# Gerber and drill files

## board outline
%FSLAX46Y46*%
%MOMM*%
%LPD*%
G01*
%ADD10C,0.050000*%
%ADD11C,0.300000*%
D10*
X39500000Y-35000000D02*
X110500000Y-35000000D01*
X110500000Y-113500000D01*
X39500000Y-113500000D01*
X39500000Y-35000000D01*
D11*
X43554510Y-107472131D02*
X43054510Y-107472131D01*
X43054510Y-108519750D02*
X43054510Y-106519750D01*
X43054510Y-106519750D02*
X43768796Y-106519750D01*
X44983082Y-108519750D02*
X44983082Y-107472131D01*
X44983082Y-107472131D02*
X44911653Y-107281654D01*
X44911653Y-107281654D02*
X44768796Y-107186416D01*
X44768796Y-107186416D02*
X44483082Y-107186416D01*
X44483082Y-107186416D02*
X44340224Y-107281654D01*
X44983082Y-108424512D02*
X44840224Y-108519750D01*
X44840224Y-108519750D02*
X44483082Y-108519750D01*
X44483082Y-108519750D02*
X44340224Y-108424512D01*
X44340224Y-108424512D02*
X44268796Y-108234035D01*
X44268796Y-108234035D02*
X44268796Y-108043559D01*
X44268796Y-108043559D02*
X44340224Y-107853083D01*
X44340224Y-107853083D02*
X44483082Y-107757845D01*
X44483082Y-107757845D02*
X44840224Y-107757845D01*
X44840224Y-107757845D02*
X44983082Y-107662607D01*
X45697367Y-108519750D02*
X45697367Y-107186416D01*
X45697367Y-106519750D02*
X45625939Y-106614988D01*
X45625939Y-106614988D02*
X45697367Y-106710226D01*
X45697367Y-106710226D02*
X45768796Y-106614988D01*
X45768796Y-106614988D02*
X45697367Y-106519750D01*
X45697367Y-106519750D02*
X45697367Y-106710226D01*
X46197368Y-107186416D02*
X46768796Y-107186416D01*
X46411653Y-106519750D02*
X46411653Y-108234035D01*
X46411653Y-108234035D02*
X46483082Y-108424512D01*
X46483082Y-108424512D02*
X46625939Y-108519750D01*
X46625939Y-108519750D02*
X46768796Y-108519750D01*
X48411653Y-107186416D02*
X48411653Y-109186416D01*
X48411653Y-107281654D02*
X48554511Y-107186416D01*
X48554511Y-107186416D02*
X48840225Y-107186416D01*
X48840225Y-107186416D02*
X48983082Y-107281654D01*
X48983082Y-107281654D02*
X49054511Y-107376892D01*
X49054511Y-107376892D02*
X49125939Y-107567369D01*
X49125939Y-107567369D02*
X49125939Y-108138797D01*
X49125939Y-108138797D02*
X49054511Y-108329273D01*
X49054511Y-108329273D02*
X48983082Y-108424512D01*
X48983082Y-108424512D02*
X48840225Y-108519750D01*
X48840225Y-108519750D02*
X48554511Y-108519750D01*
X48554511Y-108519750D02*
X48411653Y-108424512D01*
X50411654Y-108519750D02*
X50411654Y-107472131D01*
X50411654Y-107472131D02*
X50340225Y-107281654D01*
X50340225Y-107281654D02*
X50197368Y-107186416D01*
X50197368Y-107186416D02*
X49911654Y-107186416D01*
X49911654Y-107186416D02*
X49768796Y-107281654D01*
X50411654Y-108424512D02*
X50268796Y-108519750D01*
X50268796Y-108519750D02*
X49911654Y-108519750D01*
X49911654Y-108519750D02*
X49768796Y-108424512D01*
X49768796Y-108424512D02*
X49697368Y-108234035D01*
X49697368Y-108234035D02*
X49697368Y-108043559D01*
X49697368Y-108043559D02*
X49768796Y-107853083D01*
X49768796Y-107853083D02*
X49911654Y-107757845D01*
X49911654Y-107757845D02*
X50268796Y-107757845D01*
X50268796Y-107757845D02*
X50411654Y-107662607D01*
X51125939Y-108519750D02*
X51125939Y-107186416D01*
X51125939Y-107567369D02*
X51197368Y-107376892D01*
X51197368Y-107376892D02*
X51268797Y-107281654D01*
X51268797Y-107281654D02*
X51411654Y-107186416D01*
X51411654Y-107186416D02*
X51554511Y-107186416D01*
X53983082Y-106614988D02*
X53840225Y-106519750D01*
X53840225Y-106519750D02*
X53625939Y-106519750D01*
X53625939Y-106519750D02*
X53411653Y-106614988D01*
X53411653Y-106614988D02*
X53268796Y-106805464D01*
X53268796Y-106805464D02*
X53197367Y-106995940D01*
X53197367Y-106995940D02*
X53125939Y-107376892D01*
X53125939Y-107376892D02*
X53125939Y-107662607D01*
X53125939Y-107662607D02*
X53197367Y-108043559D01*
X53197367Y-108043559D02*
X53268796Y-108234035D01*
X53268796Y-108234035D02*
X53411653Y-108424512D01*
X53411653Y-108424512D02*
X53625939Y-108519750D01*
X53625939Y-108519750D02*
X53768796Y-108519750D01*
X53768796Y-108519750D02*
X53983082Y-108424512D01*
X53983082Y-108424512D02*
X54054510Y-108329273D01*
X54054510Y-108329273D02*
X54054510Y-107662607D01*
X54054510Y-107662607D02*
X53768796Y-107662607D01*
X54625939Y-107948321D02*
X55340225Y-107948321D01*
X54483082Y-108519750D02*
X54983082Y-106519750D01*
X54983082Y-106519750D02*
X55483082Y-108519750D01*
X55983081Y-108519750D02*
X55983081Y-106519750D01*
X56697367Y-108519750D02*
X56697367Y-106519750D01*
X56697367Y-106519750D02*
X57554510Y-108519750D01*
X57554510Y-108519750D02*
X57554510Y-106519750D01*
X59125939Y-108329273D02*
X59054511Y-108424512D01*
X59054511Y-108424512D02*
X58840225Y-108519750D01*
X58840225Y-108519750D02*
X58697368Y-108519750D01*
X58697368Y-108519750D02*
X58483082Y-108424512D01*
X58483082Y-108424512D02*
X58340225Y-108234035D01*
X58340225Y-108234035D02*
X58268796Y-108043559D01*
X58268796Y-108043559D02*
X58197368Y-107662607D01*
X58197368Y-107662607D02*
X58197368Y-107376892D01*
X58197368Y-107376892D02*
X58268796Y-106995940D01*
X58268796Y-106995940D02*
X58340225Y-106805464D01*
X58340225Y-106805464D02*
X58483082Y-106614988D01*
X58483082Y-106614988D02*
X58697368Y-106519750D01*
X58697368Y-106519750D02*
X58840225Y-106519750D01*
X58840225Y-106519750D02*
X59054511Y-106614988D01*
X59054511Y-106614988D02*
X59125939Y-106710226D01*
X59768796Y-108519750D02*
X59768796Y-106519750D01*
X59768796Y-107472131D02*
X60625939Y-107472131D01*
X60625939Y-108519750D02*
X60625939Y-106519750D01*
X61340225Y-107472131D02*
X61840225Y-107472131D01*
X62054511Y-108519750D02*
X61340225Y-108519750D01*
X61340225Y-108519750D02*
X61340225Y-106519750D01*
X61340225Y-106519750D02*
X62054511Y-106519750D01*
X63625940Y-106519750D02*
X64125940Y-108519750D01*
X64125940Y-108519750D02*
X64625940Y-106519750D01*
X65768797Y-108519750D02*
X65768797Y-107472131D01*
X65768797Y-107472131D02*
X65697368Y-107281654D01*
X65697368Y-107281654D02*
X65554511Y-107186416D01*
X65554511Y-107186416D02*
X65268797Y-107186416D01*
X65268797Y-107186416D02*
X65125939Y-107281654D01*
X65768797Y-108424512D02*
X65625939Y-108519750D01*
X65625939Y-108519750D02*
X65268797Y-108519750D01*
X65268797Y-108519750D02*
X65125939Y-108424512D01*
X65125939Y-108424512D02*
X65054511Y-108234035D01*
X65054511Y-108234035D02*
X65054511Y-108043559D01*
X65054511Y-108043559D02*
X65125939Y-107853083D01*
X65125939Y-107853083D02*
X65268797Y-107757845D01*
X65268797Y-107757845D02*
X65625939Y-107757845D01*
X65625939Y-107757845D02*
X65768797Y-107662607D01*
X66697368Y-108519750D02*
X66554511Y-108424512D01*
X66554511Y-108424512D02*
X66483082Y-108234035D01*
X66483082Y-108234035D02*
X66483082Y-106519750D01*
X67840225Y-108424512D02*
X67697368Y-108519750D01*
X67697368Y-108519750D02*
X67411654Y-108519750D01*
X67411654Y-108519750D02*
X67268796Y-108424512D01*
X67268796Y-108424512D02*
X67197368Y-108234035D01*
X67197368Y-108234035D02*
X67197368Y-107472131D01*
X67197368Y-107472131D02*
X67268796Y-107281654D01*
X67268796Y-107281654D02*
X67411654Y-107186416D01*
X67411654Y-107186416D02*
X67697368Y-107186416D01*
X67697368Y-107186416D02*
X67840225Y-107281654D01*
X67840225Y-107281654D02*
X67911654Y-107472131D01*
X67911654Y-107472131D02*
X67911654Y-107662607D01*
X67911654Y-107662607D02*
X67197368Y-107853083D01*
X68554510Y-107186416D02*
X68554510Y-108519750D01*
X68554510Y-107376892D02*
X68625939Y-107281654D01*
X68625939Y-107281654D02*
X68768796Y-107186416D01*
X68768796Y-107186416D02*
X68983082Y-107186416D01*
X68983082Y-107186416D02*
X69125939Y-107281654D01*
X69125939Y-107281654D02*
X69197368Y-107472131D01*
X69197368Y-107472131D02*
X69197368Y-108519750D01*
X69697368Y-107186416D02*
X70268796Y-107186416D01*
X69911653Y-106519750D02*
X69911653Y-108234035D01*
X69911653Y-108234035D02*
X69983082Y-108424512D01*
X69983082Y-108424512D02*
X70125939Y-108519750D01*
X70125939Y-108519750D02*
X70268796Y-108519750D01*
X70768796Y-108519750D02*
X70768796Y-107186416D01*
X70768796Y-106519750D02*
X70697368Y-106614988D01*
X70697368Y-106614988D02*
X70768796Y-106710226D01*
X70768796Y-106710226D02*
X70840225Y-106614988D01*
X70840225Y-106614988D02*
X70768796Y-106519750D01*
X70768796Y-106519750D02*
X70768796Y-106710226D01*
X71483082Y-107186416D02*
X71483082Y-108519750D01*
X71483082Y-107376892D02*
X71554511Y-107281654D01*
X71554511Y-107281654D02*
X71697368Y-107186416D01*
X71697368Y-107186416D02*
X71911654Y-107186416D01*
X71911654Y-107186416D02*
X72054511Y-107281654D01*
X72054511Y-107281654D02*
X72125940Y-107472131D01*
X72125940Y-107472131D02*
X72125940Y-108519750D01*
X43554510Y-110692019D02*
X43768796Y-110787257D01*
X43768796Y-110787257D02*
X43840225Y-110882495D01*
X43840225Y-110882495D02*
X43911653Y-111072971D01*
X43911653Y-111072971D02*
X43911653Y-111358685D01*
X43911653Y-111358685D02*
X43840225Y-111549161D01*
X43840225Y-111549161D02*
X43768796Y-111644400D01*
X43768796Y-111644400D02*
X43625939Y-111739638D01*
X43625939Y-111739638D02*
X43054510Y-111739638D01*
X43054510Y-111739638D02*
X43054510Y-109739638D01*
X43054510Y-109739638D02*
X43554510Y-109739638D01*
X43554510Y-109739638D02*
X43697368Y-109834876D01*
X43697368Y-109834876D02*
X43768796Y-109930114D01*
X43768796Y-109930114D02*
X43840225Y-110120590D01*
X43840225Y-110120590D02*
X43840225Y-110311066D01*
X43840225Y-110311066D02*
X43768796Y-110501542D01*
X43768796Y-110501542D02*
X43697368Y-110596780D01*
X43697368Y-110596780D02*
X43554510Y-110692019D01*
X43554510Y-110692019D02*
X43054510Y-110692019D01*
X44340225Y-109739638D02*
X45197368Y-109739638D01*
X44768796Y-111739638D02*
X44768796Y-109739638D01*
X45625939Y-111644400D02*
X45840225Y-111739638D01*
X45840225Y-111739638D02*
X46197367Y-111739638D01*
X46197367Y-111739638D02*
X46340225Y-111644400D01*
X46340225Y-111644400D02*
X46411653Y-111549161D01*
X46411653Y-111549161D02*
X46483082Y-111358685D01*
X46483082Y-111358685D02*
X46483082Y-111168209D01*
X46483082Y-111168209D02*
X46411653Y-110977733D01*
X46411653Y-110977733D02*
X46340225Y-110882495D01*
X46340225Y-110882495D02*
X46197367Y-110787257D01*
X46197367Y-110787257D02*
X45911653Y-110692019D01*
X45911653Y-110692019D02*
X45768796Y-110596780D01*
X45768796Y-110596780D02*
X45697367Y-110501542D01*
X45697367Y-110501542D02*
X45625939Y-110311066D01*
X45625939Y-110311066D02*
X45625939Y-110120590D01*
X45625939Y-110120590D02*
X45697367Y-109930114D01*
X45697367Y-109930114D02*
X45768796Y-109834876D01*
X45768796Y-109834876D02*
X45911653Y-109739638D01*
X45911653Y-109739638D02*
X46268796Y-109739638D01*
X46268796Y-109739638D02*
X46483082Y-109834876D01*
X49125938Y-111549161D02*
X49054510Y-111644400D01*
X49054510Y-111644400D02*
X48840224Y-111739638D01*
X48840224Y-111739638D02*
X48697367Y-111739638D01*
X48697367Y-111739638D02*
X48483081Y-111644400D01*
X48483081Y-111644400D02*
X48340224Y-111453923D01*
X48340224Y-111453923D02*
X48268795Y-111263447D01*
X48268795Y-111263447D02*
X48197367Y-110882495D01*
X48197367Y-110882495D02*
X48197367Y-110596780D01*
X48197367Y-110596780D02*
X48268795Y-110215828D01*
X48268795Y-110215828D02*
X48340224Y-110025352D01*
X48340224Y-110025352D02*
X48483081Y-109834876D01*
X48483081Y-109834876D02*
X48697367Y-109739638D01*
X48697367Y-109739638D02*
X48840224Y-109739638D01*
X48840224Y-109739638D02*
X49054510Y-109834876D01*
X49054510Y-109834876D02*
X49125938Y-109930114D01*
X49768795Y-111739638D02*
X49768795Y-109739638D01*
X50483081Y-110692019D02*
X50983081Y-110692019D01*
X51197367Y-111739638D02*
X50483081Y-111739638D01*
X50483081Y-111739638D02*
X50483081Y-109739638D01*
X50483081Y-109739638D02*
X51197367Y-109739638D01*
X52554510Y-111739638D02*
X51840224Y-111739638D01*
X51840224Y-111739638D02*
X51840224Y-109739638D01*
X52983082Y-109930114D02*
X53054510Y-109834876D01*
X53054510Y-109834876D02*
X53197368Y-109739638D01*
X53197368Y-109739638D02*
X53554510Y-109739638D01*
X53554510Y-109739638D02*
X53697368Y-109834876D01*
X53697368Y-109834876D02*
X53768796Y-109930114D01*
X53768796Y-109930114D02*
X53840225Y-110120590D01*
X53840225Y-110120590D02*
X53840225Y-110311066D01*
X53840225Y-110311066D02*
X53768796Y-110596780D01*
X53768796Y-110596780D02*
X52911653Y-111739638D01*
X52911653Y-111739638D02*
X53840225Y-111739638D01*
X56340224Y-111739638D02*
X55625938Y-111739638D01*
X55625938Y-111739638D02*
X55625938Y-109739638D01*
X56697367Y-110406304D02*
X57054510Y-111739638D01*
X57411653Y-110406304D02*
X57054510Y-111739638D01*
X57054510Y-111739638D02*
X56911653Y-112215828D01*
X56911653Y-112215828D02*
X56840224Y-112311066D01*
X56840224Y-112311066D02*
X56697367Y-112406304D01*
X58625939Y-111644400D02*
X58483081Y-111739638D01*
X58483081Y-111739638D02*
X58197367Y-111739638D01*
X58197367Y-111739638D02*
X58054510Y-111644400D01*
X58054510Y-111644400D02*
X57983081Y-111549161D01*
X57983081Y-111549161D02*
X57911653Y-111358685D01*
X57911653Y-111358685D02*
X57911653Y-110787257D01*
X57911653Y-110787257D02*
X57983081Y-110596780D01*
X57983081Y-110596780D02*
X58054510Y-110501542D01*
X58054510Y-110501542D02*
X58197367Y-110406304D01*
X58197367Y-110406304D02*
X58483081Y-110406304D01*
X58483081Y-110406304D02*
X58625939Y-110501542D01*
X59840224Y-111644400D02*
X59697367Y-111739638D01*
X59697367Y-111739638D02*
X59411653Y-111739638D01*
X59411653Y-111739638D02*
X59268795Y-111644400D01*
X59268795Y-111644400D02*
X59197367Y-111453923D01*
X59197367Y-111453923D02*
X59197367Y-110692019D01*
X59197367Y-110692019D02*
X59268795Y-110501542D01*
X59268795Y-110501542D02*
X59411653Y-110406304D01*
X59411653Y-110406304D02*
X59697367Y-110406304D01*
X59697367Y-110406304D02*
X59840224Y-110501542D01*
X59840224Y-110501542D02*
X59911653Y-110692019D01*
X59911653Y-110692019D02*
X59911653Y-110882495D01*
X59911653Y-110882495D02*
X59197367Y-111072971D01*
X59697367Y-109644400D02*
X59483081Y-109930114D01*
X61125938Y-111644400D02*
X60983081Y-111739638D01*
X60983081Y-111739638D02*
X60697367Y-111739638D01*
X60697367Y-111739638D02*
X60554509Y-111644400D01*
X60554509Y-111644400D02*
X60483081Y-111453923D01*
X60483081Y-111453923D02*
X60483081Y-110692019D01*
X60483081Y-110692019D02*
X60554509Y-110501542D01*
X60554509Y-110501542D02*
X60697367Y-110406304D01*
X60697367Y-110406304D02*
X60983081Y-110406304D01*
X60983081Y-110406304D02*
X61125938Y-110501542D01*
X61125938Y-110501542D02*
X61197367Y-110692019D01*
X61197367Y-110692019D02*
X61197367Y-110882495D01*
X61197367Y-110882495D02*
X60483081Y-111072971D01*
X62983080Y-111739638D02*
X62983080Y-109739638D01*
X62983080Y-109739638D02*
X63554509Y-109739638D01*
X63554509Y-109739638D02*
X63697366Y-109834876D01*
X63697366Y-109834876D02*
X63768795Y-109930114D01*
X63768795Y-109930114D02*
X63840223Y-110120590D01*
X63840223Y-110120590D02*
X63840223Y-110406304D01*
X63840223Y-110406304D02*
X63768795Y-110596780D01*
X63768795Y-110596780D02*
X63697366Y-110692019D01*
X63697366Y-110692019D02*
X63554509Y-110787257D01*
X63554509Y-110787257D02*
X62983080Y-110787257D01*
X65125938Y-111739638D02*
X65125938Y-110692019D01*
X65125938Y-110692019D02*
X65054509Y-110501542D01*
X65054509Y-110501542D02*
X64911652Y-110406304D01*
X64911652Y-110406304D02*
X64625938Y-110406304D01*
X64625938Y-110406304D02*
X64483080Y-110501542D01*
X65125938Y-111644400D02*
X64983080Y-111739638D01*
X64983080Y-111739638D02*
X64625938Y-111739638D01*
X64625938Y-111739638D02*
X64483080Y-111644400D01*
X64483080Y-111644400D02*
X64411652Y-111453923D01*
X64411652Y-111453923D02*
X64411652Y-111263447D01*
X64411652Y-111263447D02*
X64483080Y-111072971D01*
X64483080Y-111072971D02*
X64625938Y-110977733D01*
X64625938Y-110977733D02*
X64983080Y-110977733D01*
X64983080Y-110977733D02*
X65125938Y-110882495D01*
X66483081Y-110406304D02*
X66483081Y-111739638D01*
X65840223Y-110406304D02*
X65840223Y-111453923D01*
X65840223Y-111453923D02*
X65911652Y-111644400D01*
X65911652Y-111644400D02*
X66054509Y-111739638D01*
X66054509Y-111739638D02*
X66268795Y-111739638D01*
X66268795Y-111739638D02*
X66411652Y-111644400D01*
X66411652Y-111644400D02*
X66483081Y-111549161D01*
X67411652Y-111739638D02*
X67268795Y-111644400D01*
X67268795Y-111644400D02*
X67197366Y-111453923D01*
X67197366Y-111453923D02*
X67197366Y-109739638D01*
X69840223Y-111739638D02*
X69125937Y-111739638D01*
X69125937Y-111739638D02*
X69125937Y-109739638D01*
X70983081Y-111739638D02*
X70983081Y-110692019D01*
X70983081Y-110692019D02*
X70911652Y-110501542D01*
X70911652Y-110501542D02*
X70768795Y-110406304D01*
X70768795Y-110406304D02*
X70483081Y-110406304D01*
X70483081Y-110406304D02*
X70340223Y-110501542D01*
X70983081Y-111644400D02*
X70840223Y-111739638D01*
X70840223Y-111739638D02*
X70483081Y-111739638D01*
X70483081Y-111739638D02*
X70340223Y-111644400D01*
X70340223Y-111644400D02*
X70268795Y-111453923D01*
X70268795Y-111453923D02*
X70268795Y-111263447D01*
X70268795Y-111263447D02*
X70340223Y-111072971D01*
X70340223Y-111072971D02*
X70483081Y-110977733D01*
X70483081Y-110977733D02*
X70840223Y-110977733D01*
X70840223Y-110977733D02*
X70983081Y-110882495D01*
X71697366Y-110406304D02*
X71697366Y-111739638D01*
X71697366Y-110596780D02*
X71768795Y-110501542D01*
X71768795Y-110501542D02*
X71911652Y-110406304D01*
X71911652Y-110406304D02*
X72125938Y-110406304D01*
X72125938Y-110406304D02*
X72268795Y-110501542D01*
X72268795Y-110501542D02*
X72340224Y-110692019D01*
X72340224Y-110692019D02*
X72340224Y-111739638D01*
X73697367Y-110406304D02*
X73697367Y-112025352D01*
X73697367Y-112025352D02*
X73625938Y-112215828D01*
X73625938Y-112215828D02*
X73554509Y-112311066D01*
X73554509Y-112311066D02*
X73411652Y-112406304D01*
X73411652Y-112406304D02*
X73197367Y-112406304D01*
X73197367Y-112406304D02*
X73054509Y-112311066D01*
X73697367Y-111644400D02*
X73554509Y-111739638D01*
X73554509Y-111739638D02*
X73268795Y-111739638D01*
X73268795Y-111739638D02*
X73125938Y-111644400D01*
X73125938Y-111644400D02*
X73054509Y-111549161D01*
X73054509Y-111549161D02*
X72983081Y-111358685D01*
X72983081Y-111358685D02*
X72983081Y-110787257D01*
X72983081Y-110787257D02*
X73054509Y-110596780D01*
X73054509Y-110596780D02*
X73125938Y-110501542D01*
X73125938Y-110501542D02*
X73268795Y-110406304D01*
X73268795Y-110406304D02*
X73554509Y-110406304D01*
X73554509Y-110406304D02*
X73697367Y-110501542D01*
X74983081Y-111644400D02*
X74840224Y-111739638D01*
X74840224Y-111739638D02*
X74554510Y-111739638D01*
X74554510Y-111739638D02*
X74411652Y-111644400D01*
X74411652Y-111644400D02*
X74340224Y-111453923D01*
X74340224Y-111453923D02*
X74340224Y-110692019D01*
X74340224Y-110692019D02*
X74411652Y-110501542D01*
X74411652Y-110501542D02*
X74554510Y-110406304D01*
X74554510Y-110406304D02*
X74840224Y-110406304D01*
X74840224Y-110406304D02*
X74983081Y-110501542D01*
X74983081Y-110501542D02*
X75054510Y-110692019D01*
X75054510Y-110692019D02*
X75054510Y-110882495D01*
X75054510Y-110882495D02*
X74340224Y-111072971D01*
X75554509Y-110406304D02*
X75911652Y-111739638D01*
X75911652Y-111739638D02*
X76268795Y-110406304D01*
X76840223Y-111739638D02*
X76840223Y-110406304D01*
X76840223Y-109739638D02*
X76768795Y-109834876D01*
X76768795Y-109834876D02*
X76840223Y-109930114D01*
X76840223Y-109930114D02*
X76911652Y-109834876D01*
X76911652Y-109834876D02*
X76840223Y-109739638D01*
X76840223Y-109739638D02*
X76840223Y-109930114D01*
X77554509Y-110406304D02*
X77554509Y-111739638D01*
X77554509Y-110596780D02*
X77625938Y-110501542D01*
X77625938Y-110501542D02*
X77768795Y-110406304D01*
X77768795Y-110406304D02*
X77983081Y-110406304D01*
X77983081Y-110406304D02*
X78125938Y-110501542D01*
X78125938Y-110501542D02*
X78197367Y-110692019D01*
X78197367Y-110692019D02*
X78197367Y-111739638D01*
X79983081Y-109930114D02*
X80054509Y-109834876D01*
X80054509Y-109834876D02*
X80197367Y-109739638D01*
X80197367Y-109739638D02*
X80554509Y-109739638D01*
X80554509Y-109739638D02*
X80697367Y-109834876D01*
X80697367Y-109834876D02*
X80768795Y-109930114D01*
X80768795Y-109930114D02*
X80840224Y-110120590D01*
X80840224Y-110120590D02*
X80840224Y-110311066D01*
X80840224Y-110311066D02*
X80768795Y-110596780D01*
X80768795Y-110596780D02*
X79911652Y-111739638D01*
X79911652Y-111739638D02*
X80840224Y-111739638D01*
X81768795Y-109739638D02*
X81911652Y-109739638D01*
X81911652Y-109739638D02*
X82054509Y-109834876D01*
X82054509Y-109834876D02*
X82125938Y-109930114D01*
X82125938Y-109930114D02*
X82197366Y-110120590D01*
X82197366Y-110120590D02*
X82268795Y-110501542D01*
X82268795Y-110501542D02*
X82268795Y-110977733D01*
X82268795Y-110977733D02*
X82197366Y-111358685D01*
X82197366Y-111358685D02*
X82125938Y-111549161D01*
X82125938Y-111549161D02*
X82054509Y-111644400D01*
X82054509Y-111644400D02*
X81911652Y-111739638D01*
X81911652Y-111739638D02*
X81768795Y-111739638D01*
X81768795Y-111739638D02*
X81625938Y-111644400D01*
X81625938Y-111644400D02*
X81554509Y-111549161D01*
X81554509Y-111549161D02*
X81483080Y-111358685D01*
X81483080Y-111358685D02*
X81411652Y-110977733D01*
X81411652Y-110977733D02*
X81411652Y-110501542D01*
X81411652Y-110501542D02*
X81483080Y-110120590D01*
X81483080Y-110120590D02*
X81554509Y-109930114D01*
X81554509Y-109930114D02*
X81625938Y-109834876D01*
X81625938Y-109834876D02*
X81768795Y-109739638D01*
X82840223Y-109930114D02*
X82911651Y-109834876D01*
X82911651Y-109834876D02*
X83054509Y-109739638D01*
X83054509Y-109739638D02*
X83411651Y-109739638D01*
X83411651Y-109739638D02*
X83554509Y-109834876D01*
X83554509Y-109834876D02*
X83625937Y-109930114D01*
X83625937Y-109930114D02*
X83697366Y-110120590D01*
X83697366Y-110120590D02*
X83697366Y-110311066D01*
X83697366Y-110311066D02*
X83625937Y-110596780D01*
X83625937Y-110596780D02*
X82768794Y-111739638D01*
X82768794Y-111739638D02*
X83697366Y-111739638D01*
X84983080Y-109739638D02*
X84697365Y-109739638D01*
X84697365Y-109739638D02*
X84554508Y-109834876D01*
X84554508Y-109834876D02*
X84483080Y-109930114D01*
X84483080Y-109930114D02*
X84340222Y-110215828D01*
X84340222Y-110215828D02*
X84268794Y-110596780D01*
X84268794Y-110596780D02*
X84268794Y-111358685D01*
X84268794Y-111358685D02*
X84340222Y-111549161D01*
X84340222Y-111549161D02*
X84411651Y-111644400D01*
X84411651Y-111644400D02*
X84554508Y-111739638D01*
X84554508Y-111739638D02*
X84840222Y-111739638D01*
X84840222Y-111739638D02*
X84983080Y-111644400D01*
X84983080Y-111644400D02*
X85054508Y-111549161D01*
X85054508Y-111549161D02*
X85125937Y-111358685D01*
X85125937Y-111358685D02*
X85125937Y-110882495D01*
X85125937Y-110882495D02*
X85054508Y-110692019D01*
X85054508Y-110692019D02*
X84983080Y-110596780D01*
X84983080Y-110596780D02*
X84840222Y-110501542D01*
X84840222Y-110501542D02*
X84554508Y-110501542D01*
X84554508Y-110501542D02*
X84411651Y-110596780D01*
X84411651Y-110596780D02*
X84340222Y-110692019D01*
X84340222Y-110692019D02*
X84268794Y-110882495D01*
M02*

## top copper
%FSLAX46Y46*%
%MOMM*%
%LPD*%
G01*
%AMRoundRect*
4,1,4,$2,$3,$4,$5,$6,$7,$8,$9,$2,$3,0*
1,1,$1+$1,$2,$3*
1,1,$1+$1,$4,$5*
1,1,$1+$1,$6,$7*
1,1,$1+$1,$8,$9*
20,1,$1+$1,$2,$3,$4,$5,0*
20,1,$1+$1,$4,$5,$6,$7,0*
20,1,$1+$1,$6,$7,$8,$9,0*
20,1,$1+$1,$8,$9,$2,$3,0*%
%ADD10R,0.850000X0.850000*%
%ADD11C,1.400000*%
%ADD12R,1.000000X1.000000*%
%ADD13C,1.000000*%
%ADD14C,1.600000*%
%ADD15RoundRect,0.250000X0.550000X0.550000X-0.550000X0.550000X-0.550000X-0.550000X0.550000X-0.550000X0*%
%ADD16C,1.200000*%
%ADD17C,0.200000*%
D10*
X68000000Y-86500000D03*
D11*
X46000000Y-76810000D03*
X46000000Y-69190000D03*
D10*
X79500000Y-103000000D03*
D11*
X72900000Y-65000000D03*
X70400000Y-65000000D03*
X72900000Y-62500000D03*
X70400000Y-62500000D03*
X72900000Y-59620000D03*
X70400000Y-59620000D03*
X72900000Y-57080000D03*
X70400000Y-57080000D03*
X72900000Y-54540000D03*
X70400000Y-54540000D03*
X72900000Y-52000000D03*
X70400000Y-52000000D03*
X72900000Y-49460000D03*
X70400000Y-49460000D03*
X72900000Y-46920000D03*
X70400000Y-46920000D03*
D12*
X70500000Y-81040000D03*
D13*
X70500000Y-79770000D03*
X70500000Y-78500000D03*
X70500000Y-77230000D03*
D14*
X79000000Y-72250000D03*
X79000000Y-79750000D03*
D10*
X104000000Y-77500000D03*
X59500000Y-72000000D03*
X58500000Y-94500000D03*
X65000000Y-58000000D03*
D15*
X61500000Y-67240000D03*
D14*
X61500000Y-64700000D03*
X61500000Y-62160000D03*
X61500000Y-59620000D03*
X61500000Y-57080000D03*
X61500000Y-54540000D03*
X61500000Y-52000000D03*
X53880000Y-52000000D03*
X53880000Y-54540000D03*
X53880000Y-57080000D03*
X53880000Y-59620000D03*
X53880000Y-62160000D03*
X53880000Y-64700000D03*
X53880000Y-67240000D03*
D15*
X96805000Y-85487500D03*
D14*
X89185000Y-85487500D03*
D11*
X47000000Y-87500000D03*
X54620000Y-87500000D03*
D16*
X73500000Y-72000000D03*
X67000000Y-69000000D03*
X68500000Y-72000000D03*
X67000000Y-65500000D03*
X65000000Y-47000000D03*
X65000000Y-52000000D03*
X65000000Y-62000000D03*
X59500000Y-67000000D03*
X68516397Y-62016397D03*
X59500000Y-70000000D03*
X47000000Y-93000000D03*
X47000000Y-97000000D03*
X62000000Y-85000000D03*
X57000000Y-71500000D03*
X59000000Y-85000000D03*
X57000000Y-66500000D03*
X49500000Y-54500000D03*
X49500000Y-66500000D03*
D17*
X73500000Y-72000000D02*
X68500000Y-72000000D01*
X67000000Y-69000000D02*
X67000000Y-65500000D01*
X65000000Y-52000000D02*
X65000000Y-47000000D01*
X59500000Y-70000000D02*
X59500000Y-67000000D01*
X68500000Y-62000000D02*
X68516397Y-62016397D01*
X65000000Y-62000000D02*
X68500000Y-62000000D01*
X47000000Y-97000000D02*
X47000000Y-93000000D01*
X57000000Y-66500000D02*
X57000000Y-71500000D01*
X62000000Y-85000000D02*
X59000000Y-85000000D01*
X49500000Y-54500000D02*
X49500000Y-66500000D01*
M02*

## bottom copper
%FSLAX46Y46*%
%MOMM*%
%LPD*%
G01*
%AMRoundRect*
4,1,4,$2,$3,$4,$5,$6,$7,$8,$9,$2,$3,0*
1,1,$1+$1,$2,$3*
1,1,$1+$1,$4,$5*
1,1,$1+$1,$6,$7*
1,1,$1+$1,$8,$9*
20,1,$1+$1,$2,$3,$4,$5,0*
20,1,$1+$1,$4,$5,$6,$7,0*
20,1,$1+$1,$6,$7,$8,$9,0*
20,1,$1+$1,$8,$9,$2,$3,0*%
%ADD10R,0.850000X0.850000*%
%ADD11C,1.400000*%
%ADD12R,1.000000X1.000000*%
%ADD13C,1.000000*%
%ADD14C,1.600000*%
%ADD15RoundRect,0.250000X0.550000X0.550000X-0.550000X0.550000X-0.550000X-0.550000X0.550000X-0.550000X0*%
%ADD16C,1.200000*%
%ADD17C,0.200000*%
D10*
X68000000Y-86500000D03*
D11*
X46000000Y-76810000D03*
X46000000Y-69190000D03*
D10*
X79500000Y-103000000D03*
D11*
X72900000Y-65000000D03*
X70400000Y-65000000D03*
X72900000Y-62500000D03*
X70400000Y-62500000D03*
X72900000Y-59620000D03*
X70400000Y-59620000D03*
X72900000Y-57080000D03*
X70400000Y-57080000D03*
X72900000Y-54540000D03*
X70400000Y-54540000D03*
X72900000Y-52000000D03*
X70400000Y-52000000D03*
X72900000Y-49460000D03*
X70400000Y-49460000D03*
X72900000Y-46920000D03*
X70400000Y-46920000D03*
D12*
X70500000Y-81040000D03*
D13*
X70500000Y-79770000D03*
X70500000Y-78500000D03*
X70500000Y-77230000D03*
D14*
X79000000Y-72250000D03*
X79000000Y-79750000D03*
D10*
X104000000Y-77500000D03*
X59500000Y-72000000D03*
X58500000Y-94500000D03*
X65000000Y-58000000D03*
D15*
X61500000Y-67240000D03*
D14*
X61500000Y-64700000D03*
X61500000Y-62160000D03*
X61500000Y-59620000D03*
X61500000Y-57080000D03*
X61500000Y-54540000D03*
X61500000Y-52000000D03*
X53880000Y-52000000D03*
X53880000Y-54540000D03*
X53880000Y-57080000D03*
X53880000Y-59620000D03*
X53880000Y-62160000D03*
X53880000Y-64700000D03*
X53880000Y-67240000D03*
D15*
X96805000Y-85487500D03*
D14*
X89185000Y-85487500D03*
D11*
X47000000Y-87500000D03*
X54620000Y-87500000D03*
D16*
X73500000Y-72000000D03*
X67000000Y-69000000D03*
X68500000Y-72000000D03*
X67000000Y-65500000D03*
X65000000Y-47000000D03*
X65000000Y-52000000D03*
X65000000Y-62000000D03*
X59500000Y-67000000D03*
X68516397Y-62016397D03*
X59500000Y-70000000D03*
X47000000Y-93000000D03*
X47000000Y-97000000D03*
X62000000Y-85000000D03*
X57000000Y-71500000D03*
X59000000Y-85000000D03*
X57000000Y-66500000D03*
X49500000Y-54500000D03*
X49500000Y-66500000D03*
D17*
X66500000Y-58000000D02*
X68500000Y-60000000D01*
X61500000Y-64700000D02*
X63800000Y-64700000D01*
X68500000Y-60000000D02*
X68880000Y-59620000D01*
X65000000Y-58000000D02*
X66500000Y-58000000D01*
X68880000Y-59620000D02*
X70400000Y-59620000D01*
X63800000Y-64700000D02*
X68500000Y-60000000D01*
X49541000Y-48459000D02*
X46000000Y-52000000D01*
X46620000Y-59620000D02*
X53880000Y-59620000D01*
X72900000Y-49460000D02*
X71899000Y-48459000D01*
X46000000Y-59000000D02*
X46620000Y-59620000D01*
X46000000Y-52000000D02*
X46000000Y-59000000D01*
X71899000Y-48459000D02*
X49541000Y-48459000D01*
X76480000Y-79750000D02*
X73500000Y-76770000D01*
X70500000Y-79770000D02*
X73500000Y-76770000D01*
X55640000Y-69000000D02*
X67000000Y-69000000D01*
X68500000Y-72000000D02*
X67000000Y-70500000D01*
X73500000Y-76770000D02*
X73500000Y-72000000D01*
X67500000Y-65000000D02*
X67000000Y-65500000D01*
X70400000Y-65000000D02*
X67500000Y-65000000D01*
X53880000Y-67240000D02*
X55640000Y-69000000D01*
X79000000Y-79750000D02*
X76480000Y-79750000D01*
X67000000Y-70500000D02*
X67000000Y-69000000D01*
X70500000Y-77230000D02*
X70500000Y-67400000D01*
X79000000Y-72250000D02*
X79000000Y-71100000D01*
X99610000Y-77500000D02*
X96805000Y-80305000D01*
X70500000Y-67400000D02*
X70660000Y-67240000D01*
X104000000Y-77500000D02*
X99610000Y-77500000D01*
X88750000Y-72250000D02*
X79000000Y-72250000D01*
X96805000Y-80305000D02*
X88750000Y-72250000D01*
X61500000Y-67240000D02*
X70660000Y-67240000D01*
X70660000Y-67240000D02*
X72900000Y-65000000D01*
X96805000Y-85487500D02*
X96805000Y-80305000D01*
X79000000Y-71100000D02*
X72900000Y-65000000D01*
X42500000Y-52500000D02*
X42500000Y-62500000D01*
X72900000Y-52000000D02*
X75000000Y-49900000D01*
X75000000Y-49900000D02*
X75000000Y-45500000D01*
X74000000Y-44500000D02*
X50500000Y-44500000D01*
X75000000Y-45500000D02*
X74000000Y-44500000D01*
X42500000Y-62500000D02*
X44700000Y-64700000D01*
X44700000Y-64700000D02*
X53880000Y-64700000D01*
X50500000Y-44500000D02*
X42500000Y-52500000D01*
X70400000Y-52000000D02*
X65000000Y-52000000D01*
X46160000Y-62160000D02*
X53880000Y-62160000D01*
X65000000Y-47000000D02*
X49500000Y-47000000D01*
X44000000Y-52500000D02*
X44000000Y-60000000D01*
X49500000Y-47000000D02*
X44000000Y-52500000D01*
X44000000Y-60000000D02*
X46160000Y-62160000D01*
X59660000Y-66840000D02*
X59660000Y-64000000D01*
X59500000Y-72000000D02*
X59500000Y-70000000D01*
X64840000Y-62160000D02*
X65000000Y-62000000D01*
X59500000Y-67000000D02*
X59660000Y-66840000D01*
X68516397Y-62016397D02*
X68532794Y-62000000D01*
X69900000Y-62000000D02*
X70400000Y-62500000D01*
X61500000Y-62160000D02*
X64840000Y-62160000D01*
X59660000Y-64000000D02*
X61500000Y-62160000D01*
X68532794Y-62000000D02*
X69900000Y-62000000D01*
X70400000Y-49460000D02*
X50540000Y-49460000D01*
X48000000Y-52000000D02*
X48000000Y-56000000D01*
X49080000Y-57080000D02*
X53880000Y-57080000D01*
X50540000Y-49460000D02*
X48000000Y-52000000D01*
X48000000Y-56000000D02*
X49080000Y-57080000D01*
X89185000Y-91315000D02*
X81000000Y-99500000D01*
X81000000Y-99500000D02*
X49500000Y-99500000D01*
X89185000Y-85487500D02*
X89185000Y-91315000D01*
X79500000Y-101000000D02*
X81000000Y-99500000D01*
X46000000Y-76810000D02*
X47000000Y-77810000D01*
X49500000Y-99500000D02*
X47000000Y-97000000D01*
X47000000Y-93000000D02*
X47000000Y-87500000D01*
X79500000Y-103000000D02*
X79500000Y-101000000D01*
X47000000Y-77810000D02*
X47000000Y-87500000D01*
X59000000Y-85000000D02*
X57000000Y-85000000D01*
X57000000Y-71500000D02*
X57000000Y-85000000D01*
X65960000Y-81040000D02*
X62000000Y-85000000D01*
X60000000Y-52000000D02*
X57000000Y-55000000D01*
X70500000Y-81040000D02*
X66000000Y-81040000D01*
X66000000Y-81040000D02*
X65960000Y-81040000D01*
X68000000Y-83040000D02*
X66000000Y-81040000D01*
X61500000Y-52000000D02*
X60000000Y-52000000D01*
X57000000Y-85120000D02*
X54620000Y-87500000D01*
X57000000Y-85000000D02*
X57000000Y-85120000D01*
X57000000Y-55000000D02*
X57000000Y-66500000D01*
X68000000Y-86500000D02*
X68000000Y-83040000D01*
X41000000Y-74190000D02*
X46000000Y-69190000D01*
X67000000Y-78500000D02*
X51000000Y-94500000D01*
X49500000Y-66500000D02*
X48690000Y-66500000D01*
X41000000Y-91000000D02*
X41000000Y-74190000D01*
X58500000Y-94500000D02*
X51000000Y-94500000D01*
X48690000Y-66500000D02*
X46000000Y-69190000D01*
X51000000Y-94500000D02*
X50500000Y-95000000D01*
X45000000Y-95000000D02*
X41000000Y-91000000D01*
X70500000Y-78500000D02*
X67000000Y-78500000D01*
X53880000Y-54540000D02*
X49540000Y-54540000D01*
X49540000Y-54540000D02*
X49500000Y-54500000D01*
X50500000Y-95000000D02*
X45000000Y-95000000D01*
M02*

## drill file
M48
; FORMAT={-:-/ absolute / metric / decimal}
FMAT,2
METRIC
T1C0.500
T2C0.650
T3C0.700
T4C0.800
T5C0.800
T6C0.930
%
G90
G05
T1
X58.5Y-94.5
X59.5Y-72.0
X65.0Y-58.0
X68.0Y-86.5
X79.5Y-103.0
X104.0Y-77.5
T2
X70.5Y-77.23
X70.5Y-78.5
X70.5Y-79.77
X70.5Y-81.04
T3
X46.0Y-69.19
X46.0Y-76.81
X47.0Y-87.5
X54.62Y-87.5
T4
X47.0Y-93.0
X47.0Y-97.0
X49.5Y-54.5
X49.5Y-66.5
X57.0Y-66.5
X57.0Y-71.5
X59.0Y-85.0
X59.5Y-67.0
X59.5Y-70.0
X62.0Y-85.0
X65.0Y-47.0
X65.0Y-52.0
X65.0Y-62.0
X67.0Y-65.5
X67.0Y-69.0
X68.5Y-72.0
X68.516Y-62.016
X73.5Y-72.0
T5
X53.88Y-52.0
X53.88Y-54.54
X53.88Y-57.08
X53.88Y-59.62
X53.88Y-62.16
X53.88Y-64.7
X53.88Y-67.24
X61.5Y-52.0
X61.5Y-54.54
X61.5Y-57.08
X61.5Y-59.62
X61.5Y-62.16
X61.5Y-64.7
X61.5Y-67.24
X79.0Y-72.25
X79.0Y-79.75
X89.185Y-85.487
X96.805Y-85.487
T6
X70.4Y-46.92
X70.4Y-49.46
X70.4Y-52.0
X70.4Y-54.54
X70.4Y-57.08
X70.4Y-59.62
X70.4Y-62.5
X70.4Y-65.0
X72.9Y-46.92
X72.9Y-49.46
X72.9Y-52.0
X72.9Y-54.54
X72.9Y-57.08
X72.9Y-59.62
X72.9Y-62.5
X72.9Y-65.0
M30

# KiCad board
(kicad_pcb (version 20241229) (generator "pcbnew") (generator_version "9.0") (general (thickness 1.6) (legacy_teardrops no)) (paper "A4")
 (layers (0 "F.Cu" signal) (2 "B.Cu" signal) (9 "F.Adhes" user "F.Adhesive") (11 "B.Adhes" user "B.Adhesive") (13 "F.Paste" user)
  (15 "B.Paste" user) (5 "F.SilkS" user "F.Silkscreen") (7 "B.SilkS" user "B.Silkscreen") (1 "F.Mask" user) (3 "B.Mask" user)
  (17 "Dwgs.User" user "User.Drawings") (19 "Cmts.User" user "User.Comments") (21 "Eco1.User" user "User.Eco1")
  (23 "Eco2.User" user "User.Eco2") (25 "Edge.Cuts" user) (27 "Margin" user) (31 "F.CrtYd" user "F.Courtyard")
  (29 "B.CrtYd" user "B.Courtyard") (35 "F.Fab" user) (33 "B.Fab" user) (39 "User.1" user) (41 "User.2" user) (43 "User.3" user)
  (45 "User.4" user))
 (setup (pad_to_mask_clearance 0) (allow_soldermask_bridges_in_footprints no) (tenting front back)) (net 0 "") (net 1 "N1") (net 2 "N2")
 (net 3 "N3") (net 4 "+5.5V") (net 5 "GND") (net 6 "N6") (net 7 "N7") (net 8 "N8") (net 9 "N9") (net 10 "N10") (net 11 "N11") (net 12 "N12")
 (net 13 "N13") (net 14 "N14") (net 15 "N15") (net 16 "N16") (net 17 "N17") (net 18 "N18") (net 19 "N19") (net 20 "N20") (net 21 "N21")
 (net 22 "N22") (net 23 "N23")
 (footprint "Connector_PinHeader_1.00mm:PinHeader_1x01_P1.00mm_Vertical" (layer "F.Cu") (at 68 86.5 180)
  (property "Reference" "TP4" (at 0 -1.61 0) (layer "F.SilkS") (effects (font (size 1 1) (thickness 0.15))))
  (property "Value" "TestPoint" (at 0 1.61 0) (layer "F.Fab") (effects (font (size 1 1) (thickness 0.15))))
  (pad "1" thru_hole rect (at 0 0 180) (size 0.85 0.85) (drill 0.5) (layers "*.Cu" "*.Mask") (remove_unused_layers no) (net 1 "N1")))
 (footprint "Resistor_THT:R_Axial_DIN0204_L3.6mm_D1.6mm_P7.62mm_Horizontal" (layer "F.Cu") (at 46 76.81 90)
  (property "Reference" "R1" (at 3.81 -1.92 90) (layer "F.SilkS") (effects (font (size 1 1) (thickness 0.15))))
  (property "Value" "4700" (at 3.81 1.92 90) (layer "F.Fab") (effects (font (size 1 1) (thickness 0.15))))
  (pad "1" thru_hole circle (at 0 0 90) (size 1.4 1.4) (drill 0.7) (layers "*.Cu" "*.Mask") (remove_unused_layers no) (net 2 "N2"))
  (pad "2" thru_hole circle (at 7.62 0 90) (size 1.4 1.4) (drill 0.7) (layers "*.Cu" "*.Mask") (remove_unused_layers no) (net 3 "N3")))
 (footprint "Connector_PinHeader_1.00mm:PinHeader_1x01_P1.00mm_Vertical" (layer "F.Cu") (at 79.5 103 180)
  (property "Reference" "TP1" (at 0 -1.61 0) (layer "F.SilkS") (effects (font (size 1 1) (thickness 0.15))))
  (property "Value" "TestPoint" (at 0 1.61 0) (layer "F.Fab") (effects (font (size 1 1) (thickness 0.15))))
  (pad "1" thru_hole rect (at 0 0 180) (size 0.85 0.85) (drill 0.5) (layers "*.Cu" "*.Mask") (remove_unused_layers no) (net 2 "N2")))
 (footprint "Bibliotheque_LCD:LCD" (layer "F.Cu") (at 111 53.5)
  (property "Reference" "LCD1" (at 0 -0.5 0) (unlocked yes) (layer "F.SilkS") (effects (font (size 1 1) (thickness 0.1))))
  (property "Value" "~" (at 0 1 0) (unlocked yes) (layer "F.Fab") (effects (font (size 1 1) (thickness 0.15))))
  (pad "1" thru_hole circle (at -38.1 11.5 270) (size 1.4 1.4) (drill 0.93) (layers "*.Cu" "*.Mask") (remove_unused_layers no)
   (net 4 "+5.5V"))
  (pad "2" thru_hole circle (at -40.6 11.5 270) (size 1.4 1.4) (drill 0.93) (layers "*.Cu" "*.Mask") (remove_unused_layers no) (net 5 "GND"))
  (pad "3" thru_hole circle (at -38.1 9 270) (size 1.4 1.4) (drill 0.93) (layers "*.Cu" "*.Mask") (remove_unused_layers no) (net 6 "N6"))
  (pad "4" thru_hole circle (at -40.6 9 270) (size 1.4 1.4) (drill 0.93) (layers "*.Cu" "*.Mask") (remove_unused_layers no) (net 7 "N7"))
  (pad "5" thru_hole circle (at -38.1 6.12 270) (size 1.4 1.4) (drill 0.93) (layers "*.Cu" "*.Mask") (remove_unused_layers no) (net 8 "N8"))
  (pad "6" thru_hole circle (at -40.6 6.12 270) (size 1.4 1.4) (drill 0.93) (layers "*.Cu" "*.Mask") (remove_unused_layers no) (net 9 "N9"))
  (pad "7" thru_hole circle (at -38.1 3.58 270) (size 1.4 1.4) (drill 0.93) (layers "*.Cu" "*.Mask") (remove_unused_layers no)
   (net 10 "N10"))
  (pad "8" thru_hole circle (at -40.6 3.58 270) (size 1.4 1.4) (drill 0.93) (layers "*.Cu" "*.Mask") (remove_unused_layers no)
   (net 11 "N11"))
  (pad "9" thru_hole circle (at -38.1 1.04 270) (size 1.4 1.4) (drill 0.93) (layers "*.Cu" "*.Mask") (remove_unused_layers no)
   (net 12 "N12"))
  (pad "10" thru_hole circle (at -40.6 1.04 270) (size 1.4 1.4) (drill 0.93) (layers "*.Cu" "*.Mask") (remove_unused_layers no)
   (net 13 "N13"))
  (pad "11" thru_hole circle (at -38.1 -1.5 270) (size 1.4 1.4) (drill 0.93) (layers "*.Cu" "*.Mask") (remove_unused_layers no)
   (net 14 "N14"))
  (pad "12" thru_hole circle (at -40.6 -1.5 270) (size 1.4 1.4) (drill 0.93) (layers "*.Cu" "*.Mask") (remove_unused_layers no)
   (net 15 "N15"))
  (pad "13" thru_hole circle (at -38.1 -4.04 270) (size 1.4 1.4) (drill 0.93) (layers "*.Cu" "*.Mask") (remove_unused_layers no)
   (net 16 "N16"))
  (pad "14" thru_hole circle (at -40.6 -4.04 270) (size 1.4 1.4) (drill 0.93) (layers "*.Cu" "*.Mask") (remove_unused_layers no)
   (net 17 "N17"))
  (pad "15" thru_hole circle (at -38.1 -6.58 270) (size 1.4 1.4) (drill 0.93) (layers "*.Cu" "*.Mask") (remove_unused_layers no)
   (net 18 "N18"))
  (pad "16" thru_hole circle (at -40.6 -6.58 270) (size 1.4 1.4) (drill 0.93) (layers "*.Cu" "*.Mask") (remove_unused_layers no)
   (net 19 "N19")))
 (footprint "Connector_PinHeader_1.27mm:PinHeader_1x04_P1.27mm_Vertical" (layer "F.Cu") (at 70.5 81.04 180)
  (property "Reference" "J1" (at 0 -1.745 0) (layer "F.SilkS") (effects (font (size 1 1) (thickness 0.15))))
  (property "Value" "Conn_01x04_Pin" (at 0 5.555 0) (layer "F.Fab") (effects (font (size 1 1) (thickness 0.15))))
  (pad "1" thru_hole rect (at 0 0 180) (size 1 1) (drill 0.65) (layers "*.Cu" "*.Mask") (remove_unused_layers no) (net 1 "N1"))
  (pad "2" thru_hole circle (at 0 1.27 180) (size 1 1) (drill 0.65) (layers "*.Cu" "*.Mask") (remove_unused_layers no) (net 5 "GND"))
  (pad "3" thru_hole circle (at 0 2.54 180) (size 1 1) (drill 0.65) (layers "*.Cu" "*.Mask") (remove_unused_layers no) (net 3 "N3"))
  (pad "4" thru_hole circle (at 0 3.81 180) (size 1 1) (drill 0.65) (layers "*.Cu" "*.Mask") (remove_unused_layers no) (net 4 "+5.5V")))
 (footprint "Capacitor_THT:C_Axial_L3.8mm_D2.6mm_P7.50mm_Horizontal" (layer "F.Cu") (at 79 72.25 -90)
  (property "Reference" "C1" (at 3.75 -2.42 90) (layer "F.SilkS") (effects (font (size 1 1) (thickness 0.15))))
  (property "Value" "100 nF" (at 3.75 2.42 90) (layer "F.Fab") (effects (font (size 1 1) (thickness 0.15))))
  (pad "1" thru_hole circle (at 0 0 270) (size 1.6 1.6) (drill 0.8) (layers "*.Cu" "*.Mask") (remove_unused_layers no) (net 4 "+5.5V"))
  (pad "2" thru_hole circle (at 7.5 0 270) (size 1.6 1.6) (drill 0.8) (layers "*.Cu" "*.Mask") (remove_unused_layers no) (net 5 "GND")))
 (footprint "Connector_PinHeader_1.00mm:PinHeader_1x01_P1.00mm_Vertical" (layer "F.Cu") (at 104 77.5 180)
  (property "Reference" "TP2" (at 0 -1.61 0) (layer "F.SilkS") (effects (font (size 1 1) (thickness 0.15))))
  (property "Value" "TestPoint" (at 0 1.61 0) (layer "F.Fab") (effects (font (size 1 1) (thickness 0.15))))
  (pad "1" thru_hole rect (at 0 0 180) (size 0.85 0.85) (drill 0.5) (layers "*.Cu" "*.Mask") (remove_unused_layers no) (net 4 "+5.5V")))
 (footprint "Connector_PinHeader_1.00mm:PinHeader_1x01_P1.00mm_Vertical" (layer "F.Cu") (at 59.5 72 180)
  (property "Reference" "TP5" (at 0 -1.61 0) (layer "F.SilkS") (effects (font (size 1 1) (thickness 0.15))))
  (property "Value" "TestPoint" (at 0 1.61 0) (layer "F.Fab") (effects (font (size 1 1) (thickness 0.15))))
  (pad "1" thru_hole rect (at 0 0 180) (size 0.85 0.85) (drill 0.5) (layers "*.Cu" "*.Mask") (remove_unused_layers no) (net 7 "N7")))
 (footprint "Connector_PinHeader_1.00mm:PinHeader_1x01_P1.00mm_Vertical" (layer "F.Cu") (at 58.5 94.5)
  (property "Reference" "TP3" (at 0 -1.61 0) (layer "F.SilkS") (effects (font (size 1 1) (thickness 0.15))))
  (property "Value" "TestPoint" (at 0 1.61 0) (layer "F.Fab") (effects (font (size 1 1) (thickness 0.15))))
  (pad "1" thru_hole rect (at 0 0) (size 0.85 0.85) (drill 0.5) (layers "*.Cu" "*.Mask") (remove_unused_layers no) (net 3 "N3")))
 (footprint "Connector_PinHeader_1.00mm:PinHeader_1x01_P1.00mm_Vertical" (layer "F.Cu") (at 65 58 180)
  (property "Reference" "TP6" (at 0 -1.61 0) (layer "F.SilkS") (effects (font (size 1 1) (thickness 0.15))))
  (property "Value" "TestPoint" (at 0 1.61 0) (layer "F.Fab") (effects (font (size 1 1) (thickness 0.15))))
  (pad "1" thru_hole rect (at 0 0 180) (size 0.85 0.85) (drill 0.5) (layers "*.Cu" "*.Mask") (remove_unused_layers no) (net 9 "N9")))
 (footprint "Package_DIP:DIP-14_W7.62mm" (layer "F.Cu") (at 61.5 67.24 180)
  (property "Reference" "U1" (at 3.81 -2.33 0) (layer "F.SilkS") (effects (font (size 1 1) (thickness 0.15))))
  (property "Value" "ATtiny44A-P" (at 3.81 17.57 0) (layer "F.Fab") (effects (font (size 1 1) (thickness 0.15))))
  (pad "1" thru_hole roundrect (at 0 0 180) (size 1.6 1.6) (drill 0.8) (layers "*.Cu" "*.Mask") (remove_unused_layers no)
   (roundrect_rratio 0.15625) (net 4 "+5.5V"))
  (pad "2" thru_hole circle (at 0 2.54 180) (size 1.6 1.6) (drill 0.8) (layers "*.Cu" "*.Mask") (remove_unused_layers no) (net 9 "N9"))
  (pad "3" thru_hole circle (at 0 5.08 180) (size 1.6 1.6) (drill 0.8) (layers "*.Cu" "*.Mask") (remove_unused_layers no) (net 7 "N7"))
  (pad "4" thru_hole circle (at 0 7.62 180) (size 1.6 1.6) (drill 0.8) (layers "*.Cu" "*.Mask") (remove_unused_layers no) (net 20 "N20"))
  (pad "5" thru_hole circle (at 0 10.16 180) (size 1.6 1.6) (drill 0.8) (layers "*.Cu" "*.Mask") (remove_unused_layers no) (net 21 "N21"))
  (pad "6" thru_hole circle (at 0 12.7 180) (size 1.6 1.6) (drill 0.8) (layers "*.Cu" "*.Mask") (remove_unused_layers no) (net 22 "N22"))
  (pad "7" thru_hole circle (at 0 15.24 180) (size 1.6 1.6) (drill 0.8) (layers "*.Cu" "*.Mask") (remove_unused_layers no) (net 1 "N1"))
  (pad "8" thru_hole circle (at 7.62 15.24 180) (size 1.6 1.6) (drill 0.8) (layers "*.Cu" "*.Mask") (remove_unused_layers no) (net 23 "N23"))
  (pad "9" thru_hole circle (at 7.62 12.7 180) (size 1.6 1.6) (drill 0.8) (layers "*.Cu" "*.Mask") (remove_unused_layers no) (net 3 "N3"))
  (pad "10" thru_hole circle (at 7.62 10.16 180) (size 1.6 1.6) (drill 0.8) (layers "*.Cu" "*.Mask") (remove_unused_layers no)
   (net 17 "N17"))
  (pad "11" thru_hole circle (at 7.62 7.62 180) (size 1.6 1.6) (drill 0.8) (layers "*.Cu" "*.Mask") (remove_unused_layers no) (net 16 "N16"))
  (pad "12" thru_hole circle (at 7.62 5.08 180) (size 1.6 1.6) (drill 0.8) (layers "*.Cu" "*.Mask") (remove_unused_layers no) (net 15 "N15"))
  (pad "13" thru_hole circle (at 7.62 2.54 180) (size 1.6 1.6) (drill 0.8) (layers "*.Cu" "*.Mask") (remove_unused_layers no) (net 14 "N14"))
  (pad "14" thru_hole circle (at 7.62 0 180) (size 1.6 1.6) (drill 0.8) (layers "*.Cu" "*.Mask") (remove_unused_layers no) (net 5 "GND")))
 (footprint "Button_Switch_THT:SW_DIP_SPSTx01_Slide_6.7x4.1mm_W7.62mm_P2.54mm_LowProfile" (layer "F.Cu") (at 96.805 85.4875 180)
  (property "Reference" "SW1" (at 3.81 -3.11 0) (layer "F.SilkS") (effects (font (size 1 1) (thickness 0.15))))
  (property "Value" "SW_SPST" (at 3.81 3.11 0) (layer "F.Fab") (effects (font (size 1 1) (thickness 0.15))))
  (pad "1" thru_hole roundrect (at 0 0 180) (size 1.6 1.6) (drill 0.8) (layers "*.Cu" "*.Mask") (remove_unused_layers no)
   (roundrect_rratio 0.15625) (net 4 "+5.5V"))
  (pad "2" thru_hole circle (at 7.62 0 180) (size 1.6 1.6) (drill 0.8) (layers "*.Cu" "*.Mask") (remove_unused_layers no) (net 2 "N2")))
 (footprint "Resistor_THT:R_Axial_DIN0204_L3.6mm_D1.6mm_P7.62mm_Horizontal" (layer "F.Cu") (at 47 87.5)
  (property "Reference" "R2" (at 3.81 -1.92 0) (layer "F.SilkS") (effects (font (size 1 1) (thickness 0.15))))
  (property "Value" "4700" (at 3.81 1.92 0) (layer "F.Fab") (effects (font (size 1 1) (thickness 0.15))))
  (pad "1" thru_hole circle (at 0 0) (size 1.4 1.4) (drill 0.7) (layers "*.Cu" "*.Mask") (remove_unused_layers no) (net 2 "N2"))
  (pad "2" thru_hole circle (at 7.62 0) (size 1.4 1.4) (drill 0.7) (layers "*.Cu" "*.Mask") (remove_unused_layers no) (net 1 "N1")))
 (gr_rect (start 39.5 35) (end 110.5 113.5) (stroke (width 0.05) (type default)) (fill no) (layer "Edge.Cuts"))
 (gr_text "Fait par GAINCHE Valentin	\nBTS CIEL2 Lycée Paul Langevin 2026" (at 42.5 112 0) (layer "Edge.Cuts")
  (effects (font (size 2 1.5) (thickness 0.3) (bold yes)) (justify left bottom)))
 (segment (start 66.5 58) (end 68.5 60) (width 0.2) (layer "B.Cu") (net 9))
 (segment (start 61.5 64.7) (end 63.8 64.7) (width 0.2) (layer "B.Cu") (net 9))
 (segment (start 68.5 60) (end 68.88 59.62) (width 0.2) (layer "B.Cu") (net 9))
 (segment (start 65 58) (end 66.5 58) (width 0.2) (layer "B.Cu") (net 9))
 (segment (start 68.88 59.62) (end 70.4 59.62) (width 0.2) (layer "B.Cu") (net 9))
 (segment (start 63.8 64.7) (end 68.5 60) (width 0.2) (layer "B.Cu") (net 9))
 (segment (start 49.541 48.459) (end 46 52) (width 0.2) (layer "B.Cu") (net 16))
 (segment (start 46.62 59.62) (end 53.88 59.62) (width 0.2) (layer "B.Cu") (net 16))
 (segment (start 72.9 49.46) (end 71.899 48.459) (width 0.2) (layer "B.Cu") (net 16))
 (segment (start 46 59) (end 46.62 59.62) (width 0.2) (layer "B.Cu") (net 16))
 (segment (start 46 52) (end 46 59) (width 0.2) (layer "B.Cu") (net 16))
 (segment (start 71.899 48.459) (end 49.541 48.459) (width 0.2) (layer "B.Cu") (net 16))
 (segment (start 73.5 72) (end 68.5 72) (width 0.2) (layer "F.Cu") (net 5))
 (segment (start 67 69) (end 67 65.5) (width 0.2) (layer "F.Cu") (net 5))
 (via (at 73.5 72) (size 1.2) (drill 0.8) (layers "F.Cu" "B.Cu") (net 5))
 (via (at 67 69) (size 1.2) (drill 0.8) (layers "F.Cu" "B.Cu") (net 5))
 (via (at 68.5 72) (size 1.2) (drill 0.8) (layers "F.Cu" "B.Cu") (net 5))
 (via (at 67 65.5) (size 1.2) (drill 0.8) (layers "F.Cu" "B.Cu") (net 5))
 (segment (start 76.48 79.75) (end 73.5 76.77) (width 0.2) (layer "B.Cu") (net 5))
 (segment (start 70.5 79.77) (end 73.5 76.77) (width 0.2) (layer "B.Cu") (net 5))
 (segment (start 55.64 69) (end 67 69) (width 0.2) (layer "B.Cu") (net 5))
 (segment (start 68.5 72) (end 67 70.5) (width 0.2) (layer "B.Cu") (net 5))
 (segment (start 73.5 76.77) (end 73.5 72) (width 0.2) (layer "B.Cu") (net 5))
 (segment (start 67.5 65) (end 67 65.5) (width 0.2) (layer "B.Cu") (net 5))
 (segment (start 70.4 65) (end 67.5 65) (width 0.2) (layer "B.Cu") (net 5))
 (segment (start 53.88 67.24) (end 55.64 69) (width 0.2) (layer "B.Cu") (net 5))
 (segment (start 79 79.75) (end 76.48 79.75) (width 0.2) (layer "B.Cu") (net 5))
 (segment (start 67 70.5) (end 67 69) (width 0.2) (layer "B.Cu") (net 5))
 (segment (start 70.5 77.23) (end 70.5 67.4) (width 0.2) (layer "B.Cu") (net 4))
 (segment (start 79 72.25) (end 79 71.1) (width 0.2) (layer "B.Cu") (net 4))
 (segment (start 99.61 77.5) (end 96.805 80.305) (width 0.2) (layer "B.Cu") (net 4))
 (segment (start 70.5 67.4) (end 70.66 67.24) (width 0.2) (layer "B.Cu") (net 4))
 (segment (start 104 77.5) (end 99.61 77.5) (width 0.2) (layer "B.Cu") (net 4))
 (segment (start 88.75 72.25) (end 79 72.25) (width 0.2) (layer "B.Cu") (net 4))
 (segment (start 96.805 80.305) (end 88.75 72.25) (width 0.2) (layer "B.Cu") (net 4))
 (segment (start 61.5 67.24) (end 70.66 67.24) (width 0.2) (layer "B.Cu") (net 4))
 (segment (start 70.66 67.24) (end 72.9 65) (width 0.2) (layer "B.Cu") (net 4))
 (segment (start 96.805 85.4875) (end 96.805 80.305) (width 0.2) (layer "B.Cu") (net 4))
 (segment (start 79 71.1) (end 72.9 65) (width 0.2) (layer "B.Cu") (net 4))
 (segment (start 42.5 52.5) (end 42.5 62.5) (width 0.2) (layer "B.Cu") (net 14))
 (segment (start 72.9 52) (end 75 49.9) (width 0.2) (layer "B.Cu") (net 14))
 (segment (start 75 49.9) (end 75 45.5) (width 0.2) (layer "B.Cu") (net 14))
 (segment (start 74 44.5) (end 50.5 44.5) (width 0.2) (layer "B.Cu") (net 14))
 (segment (start 75 45.5) (end 74 44.5) (width 0.2) (layer "B.Cu") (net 14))
 (segment (start 42.5 62.5) (end 44.7 64.7) (width 0.2) (layer "B.Cu") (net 14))
 (segment (start 44.7 64.7) (end 53.88 64.7) (width 0.2) (layer "B.Cu") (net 14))
 (segment (start 50.5 44.5) (end 42.5 52.5) (width 0.2) (layer "B.Cu") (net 14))
 (segment (start 65 52) (end 65 47) (width 0.2) (layer "F.Cu") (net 15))
 (via (at 65 47) (size 1.2) (drill 0.8) (layers "F.Cu" "B.Cu") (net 15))
 (via (at 65 52) (size 1.2) (drill 0.8) (layers "F.Cu" "B.Cu") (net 15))
 (segment (start 70.4 52) (end 65 52) (width 0.2) (layer "B.Cu") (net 15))
 (segment (start 46.16 62.16) (end 53.88 62.16) (width 0.2) (layer "B.Cu") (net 15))
 (segment (start 65 47) (end 49.5 47) (width 0.2) (layer "B.Cu") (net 15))
 (segment (start 44 52.5) (end 44 60) (width 0.2) (layer "B.Cu") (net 15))
 (segment (start 49.5 47) (end 44 52.5) (width 0.2) (layer "B.Cu") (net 15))
 (segment (start 44 60) (end 46.16 62.16) (width 0.2) (layer "B.Cu") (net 15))
 (segment (start 59.5 70) (end 59.5 67) (width 0.2) (layer "F.Cu") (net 7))
 (segment (start 68.5 62) (end 68.516397 62.016397) (width 0.2) (layer "F.Cu") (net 7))
 (segment (start 65 62) (end 68.5 62) (width 0.2) (layer "F.Cu") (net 7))
 (via (at 65 62) (size 1.2) (drill 0.8) (layers "F.Cu" "B.Cu") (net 7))
 (via (at 59.5 67) (size 1.2) (drill 0.8) (layers "F.Cu" "B.Cu") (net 7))
 (via (at 68.516397 62.016397) (size 1.2) (drill 0.8) (layers "F.Cu" "B.Cu") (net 7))
 (via (at 59.5 70) (size 1.2) (drill 0.8) (layers "F.Cu" "B.Cu") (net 7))
 (segment (start 59.66 66.84) (end 59.66 64) (width 0.2) (layer "B.Cu") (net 7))
 (segment (start 59.5 72) (end 59.5 70) (width 0.2) (layer "B.Cu") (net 7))
 (segment (start 64.84 62.16) (end 65 62) (width 0.2) (layer "B.Cu") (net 7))
 (segment (start 59.5 67) (end 59.66 66.84) (width 0.2) (layer "B.Cu") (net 7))
 (segment (start 68.516397 62.016397) (end 68.532794 62) (width 0.2) (layer "B.Cu") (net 7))
 (segment (start 69.9 62) (end 70.4 62.5) (width 0.2) (layer "B.Cu") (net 7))
 (segment (start 61.5 62.16) (end 64.84 62.16) (width 0.2) (layer "B.Cu") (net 7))
 (segment (start 59.66 64) (end 61.5 62.16) (width 0.2) (layer "B.Cu") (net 7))
 (segment (start 68.532794 62) (end 69.9 62) (width 0.2) (layer "B.Cu") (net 7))
 (segment (start 70.4 49.46) (end 50.54 49.46) (width 0.2) (layer "B.Cu") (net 17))
 (segment (start 48 52) (end 48 56) (width 0.2) (layer "B.Cu") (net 17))
 (segment (start 49.08 57.08) (end 53.88 57.08) (width 0.2) (layer "B.Cu") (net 17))
 (segment (start 50.54 49.46) (end 48 52) (width 0.2) (layer "B.Cu") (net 17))
 (segment (start 48 56) (end 49.08 57.08) (width 0.2) (layer "B.Cu") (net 17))
 (segment (start 47 97) (end 47 93) (width 0.2) (layer "F.Cu") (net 2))
 (via (at 47 93) (size 1.2) (drill 0.8) (layers "F.Cu" "B.Cu") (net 2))
 (via (at 47 97) (size 1.2) (drill 0.8) (layers "F.Cu" "B.Cu") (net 2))
 (segment (start 89.185 91.315) (end 81 99.5) (width 0.2) (layer "B.Cu") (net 2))
 (segment (start 81 99.5) (end 49.5 99.5) (width 0.2) (layer "B.Cu") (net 2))
 (segment (start 89.185 85.4875) (end 89.185 91.315) (width 0.2) (layer "B.Cu") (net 2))
 (segment (start 79.5 101) (end 81 99.5) (width 0.2) (layer "B.Cu") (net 2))
 (segment (start 46 76.81) (end 47 77.81) (width 0.2) (layer "B.Cu") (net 2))
 (segment (start 49.5 99.5) (end 47 97) (width 0.2) (layer "B.Cu") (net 2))
 (segment (start 47 93) (end 47 87.5) (width 0.2) (layer "B.Cu") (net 2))
 (segment (start 79.5 103) (end 79.5 101) (width 0.2) (layer "B.Cu") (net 2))
 (segment (start 47 77.81) (end 47 87.5) (width 0.2) (layer "B.Cu") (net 2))
 (segment (start 57 66.5) (end 57 71.5) (width 0.2) (layer "F.Cu") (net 1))
 (segment (start 62 85) (end 59 85) (width 0.2) (layer "F.Cu") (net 1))
 (via (at 62 85) (size 1.2) (drill 0.8) (layers "F.Cu" "B.Cu") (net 1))
 (via (at 57 71.5) (size 1.2) (drill 0.8) (layers "F.Cu" "B.Cu") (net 1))
 (via (at 59 85) (size 1.2) (drill 0.8) (layers "F.Cu" "B.Cu") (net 1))
 (via (at 57 66.5) (size 1.2) (drill 0.8) (layers "F.Cu" "B.Cu") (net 1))
 (segment (start 59 85) (end 57 85) (width 0.2) (layer "B.Cu") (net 1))
 (segment (start 57 71.5) (end 57 85) (width 0.2) (layer "B.Cu") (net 1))
 (segment (start 65.96 81.04) (end 62 85) (width 0.2) (layer "B.Cu") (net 1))
 (segment (start 60 52) (end 57 55) (width 0.2) (layer "B.Cu") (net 1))
 (segment (start 70.5 81.04) (end 66 81.04) (width 0.2) (layer "B.Cu") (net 1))
 (segment (start 66 81.04) (end 65.96 81.04) (width 0.2) (layer "B.Cu") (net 1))
 (segment (start 68 83.04) (end 66 81.04) (width 0.2) (layer "B.Cu") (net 1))
 (segment (start 61.5 52) (end 60 52) (width 0.2) (layer "B.Cu") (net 1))
 (segment (start 57 85.12) (end 54.62 87.5) (width 0.2) (layer "B.Cu") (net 1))
 (segment (start 57 85) (end 57 85.12) (width 0.2) (layer "B.Cu") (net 1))
 (segment (start 57 55) (end 57 66.5) (width 0.2) (layer "B.Cu") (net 1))
 (segment (start 68 86.5) (end 68 83.04) (width 0.2) (layer "B.Cu") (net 1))
 (segment (start 49.5 54.5) (end 49.5 66.5) (width 0.2) (layer "F.Cu") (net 3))
 (via (at 49.5 54.5) (size 1.2) (drill 0.8) (layers "F.Cu" "B.Cu") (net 3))
 (via (at 49.5 66.5) (size 1.2) (drill 0.8) (layers "F.Cu" "B.Cu") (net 3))
 (segment (start 41 74.19) (end 46 69.19) (width 0.2) (layer "B.Cu") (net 3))
 (segment (start 67 78.5) (end 51 94.5) (width 0.2) (layer "B.Cu") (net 3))
 (segment (start 49.5 66.5) (end 48.69 66.5) (width 0.2) (layer "B.Cu") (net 3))
 (segment (start 41 91) (end 41 74.19) (width 0.2) (layer "B.Cu") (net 3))
 (segment (start 58.5 94.5) (end 51 94.5) (width 0.2) (layer "B.Cu") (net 3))
 (segment (start 48.69 66.5) (end 46 69.19) (width 0.2) (layer "B.Cu") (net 3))
 (segment (start 51 94.5) (end 50.5 95) (width 0.2) (layer "B.Cu") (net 3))
 (segment (start 45 95) (end 41 91) (width 0.2) (layer "B.Cu") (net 3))
 (segment (start 70.5 78.5) (end 67 78.5) (width 0.2) (layer "B.Cu") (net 3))
 (segment (start 53.88 54.54) (end 49.54 54.54) (width 0.2) (layer "B.Cu") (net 3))
 (segment (start 49.54 54.54) (end 49.5 54.5) (width 0.2) (layer "B.Cu") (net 3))
 (segment (start 50.5 95) (end 45 95) (width 0.2) (layer "B.Cu") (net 3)))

